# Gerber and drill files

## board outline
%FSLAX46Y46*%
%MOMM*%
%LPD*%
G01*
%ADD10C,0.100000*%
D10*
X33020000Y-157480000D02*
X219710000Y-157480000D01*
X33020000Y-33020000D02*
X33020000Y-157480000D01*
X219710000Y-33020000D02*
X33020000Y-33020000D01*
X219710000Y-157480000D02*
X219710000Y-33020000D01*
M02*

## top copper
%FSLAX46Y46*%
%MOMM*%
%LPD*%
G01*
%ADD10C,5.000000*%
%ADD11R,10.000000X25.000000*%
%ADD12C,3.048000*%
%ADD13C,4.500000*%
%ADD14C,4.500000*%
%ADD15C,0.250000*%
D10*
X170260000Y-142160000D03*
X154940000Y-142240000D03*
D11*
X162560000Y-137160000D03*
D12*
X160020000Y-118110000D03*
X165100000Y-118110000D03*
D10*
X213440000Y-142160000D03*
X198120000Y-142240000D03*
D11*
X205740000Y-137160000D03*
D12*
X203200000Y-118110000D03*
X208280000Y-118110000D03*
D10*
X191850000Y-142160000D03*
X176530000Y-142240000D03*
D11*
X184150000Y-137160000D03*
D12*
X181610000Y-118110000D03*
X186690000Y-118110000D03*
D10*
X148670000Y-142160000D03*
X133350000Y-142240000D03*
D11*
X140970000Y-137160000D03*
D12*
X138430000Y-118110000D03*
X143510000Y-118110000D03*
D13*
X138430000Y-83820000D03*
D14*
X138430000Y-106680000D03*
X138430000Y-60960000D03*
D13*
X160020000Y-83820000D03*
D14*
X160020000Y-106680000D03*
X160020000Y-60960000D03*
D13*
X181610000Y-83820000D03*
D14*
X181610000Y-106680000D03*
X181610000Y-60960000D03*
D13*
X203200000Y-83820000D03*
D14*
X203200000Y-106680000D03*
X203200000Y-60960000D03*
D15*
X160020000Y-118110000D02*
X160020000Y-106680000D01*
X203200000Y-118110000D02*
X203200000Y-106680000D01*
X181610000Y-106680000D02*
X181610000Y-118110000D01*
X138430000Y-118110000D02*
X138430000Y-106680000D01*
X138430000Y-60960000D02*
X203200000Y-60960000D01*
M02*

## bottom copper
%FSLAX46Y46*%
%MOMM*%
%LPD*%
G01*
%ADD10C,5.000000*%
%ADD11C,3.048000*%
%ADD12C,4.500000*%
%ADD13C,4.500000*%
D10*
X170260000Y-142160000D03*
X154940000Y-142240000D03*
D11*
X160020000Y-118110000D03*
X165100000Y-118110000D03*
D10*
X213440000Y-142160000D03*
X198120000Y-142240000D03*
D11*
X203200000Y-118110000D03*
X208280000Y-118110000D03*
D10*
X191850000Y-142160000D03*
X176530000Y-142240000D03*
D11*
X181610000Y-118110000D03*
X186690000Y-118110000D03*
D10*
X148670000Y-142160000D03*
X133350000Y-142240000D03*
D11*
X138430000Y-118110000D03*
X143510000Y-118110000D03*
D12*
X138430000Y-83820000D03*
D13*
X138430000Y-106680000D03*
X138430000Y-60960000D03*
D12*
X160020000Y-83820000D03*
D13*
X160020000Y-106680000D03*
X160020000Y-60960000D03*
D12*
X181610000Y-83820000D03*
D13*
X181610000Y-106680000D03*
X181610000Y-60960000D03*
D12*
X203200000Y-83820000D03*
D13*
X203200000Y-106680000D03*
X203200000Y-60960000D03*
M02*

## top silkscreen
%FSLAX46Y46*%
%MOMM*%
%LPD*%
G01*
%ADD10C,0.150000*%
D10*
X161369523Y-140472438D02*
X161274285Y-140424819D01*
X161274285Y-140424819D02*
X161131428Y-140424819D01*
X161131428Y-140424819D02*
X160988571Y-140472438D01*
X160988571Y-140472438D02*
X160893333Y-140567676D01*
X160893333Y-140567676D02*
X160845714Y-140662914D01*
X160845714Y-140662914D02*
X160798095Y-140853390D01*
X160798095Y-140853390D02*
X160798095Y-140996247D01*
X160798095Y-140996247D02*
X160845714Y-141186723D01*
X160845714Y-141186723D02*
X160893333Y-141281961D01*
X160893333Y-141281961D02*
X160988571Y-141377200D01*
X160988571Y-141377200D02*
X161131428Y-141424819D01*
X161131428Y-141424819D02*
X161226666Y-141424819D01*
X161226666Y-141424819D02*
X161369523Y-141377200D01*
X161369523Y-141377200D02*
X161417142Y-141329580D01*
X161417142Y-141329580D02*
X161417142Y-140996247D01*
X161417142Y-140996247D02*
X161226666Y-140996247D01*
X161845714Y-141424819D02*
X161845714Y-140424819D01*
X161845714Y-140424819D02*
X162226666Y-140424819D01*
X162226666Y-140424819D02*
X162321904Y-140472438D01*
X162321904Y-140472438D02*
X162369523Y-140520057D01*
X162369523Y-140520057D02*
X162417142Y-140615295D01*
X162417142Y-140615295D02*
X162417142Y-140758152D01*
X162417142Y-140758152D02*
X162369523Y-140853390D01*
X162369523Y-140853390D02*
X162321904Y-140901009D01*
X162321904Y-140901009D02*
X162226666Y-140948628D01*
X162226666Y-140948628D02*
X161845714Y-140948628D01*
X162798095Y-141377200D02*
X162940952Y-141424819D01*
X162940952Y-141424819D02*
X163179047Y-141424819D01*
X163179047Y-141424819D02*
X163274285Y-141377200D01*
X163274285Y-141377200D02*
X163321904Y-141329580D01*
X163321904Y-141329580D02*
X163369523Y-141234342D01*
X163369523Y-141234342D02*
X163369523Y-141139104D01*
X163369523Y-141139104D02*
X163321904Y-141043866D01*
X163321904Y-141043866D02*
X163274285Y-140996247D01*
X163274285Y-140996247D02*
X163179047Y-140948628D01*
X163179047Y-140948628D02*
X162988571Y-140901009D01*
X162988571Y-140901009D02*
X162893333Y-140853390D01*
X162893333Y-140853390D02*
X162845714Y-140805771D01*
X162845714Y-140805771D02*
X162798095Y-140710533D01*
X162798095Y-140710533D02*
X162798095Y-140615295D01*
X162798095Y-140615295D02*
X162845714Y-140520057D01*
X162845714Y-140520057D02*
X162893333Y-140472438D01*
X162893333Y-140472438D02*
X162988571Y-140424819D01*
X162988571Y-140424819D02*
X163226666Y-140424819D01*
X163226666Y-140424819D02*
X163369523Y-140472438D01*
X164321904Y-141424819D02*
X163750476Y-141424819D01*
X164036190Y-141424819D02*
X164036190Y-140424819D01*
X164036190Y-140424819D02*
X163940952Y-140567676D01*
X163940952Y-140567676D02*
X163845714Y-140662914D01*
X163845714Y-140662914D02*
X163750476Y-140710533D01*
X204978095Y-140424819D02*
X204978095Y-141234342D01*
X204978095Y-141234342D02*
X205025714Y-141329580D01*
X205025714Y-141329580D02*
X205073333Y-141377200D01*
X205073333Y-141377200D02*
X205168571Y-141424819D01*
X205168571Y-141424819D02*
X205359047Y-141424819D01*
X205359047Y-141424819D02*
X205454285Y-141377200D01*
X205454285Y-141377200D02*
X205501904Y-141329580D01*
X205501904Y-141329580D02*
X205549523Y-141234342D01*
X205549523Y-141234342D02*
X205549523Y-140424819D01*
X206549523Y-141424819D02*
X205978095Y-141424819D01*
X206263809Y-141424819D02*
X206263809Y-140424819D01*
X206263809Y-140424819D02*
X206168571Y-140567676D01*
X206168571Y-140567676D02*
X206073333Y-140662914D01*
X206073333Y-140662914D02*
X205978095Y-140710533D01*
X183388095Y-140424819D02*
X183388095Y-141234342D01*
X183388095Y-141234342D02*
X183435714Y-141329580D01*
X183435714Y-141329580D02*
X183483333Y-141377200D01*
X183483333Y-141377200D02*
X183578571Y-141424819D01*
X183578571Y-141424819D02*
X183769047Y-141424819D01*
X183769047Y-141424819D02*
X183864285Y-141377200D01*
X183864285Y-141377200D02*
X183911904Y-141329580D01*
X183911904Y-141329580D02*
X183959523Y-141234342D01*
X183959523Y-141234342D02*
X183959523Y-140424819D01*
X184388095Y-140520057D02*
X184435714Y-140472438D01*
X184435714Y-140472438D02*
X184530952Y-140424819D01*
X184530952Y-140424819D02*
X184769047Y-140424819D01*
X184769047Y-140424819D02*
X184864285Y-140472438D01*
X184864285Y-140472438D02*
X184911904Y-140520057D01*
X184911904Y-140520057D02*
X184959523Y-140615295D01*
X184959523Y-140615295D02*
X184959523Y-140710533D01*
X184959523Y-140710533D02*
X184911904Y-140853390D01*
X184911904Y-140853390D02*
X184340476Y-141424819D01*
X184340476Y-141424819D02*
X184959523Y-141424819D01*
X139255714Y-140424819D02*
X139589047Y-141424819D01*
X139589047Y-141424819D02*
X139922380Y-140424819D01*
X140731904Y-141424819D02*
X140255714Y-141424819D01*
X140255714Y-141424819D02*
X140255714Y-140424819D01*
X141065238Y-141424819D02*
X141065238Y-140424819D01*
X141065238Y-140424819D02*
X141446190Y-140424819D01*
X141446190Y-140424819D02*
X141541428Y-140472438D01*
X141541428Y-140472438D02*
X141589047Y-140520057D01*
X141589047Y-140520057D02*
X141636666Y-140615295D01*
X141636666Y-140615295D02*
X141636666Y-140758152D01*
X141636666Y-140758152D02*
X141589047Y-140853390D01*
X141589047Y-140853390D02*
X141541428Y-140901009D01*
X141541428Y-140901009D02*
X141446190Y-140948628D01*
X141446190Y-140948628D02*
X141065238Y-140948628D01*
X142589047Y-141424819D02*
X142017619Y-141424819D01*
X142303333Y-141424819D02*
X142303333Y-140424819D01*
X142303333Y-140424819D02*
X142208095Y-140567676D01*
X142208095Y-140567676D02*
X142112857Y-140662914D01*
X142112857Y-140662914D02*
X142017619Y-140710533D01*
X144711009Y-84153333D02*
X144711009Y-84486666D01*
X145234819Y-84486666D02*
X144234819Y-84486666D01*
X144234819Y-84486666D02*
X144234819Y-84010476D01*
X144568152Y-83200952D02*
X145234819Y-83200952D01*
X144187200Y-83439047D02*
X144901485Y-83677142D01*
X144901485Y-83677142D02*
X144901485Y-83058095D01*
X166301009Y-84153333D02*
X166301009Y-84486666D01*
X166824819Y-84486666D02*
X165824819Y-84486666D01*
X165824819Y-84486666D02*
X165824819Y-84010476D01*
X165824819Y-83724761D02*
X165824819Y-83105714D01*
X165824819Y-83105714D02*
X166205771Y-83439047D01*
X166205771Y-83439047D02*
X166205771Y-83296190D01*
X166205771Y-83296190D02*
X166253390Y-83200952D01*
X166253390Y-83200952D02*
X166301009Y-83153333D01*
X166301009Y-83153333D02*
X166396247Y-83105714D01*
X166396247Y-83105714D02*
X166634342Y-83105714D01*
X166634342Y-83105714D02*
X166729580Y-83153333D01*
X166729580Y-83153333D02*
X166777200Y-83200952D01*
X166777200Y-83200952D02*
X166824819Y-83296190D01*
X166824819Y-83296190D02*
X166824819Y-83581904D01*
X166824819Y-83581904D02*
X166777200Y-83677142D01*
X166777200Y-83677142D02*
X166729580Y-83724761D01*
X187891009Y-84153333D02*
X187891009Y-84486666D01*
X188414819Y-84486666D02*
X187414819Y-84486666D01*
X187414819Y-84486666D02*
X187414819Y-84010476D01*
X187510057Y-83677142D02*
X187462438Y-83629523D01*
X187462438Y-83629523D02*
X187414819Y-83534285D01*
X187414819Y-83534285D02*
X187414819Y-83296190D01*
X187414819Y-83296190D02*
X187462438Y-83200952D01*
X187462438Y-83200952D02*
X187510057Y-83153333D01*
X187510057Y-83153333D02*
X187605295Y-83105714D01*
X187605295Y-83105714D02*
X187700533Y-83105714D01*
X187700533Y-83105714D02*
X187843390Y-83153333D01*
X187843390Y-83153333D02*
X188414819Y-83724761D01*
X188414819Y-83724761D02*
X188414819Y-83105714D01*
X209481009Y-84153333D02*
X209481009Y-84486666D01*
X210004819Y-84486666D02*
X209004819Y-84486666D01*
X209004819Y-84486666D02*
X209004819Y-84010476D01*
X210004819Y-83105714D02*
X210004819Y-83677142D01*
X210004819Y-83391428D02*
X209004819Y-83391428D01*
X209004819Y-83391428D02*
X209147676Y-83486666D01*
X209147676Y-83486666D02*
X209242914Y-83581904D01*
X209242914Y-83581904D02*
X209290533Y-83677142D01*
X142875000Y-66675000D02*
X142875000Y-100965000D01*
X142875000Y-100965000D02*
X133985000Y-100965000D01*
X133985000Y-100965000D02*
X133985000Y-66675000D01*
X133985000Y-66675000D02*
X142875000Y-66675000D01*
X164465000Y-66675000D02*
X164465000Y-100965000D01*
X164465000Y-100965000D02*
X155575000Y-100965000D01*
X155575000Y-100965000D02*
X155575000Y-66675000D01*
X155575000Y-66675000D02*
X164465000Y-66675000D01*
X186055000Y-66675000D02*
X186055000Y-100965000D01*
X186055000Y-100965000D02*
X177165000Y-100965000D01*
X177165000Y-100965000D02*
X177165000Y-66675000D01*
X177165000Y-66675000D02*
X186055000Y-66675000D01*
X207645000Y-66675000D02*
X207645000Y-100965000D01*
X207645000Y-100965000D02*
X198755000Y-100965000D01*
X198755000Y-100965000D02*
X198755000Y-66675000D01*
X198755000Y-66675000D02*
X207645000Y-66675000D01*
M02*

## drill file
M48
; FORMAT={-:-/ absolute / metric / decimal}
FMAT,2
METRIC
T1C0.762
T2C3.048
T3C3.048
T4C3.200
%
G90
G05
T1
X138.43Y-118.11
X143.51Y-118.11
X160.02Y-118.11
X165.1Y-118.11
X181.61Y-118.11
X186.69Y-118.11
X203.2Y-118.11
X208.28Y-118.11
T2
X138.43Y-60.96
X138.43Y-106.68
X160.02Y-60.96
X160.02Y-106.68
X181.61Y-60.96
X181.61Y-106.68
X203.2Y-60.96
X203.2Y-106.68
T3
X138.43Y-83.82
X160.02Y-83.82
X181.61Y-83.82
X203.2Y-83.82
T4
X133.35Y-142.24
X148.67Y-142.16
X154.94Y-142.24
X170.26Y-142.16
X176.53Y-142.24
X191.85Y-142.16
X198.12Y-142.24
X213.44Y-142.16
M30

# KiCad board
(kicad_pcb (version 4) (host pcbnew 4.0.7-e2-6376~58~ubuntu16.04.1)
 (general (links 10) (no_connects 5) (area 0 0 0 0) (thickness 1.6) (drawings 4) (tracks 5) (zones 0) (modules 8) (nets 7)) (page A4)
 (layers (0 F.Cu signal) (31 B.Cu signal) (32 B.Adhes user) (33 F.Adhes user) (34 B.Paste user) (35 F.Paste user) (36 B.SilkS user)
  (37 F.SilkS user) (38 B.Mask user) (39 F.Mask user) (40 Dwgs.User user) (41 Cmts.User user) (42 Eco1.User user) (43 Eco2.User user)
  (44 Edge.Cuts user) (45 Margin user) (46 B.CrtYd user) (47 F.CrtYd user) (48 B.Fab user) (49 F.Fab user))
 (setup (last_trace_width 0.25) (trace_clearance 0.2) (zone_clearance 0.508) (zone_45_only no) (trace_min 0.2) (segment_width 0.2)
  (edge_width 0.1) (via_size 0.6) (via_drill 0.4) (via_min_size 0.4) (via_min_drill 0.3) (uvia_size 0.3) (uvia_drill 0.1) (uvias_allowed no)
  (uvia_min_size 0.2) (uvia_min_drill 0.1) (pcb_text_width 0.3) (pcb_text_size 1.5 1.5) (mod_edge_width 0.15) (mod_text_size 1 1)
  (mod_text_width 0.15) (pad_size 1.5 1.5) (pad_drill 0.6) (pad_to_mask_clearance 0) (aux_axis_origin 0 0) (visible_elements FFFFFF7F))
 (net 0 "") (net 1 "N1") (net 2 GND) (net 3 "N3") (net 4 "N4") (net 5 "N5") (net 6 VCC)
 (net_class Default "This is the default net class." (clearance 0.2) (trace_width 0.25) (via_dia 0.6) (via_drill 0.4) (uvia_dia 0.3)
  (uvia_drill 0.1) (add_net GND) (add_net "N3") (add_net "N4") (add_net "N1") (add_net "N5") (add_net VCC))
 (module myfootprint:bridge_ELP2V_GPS (layer F.Cu) (at 162.56 137.16)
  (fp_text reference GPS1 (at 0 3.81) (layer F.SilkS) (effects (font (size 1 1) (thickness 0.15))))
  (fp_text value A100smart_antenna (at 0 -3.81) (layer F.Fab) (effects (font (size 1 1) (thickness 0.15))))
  (pad "" np_thru_hole circle (at 7.7 5) (size 5 5) (drill 3.2) (layers *.Cu *.Mask))
  (pad "" np_thru_hole circle (at -7.62 5.08) (size 5 5) (drill 3.2) (layers *.Cu *.Mask))
  (pad "" connect rect (at 0 0) (size 10 25) (layers F.Cu F.Mask))
  (pad 10 thru_hole circle (at -2.54 -19.05) (size 3.048 3.048) (drill 0.762) (layers *.Mask F.Cu) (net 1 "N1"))
  (pad 11 thru_hole circle (at 2.54 -19.05) (size 3.048 3.048) (drill 0.762) (layers *.Mask B.Cu) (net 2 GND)))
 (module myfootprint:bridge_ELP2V (layer F.Cu) (at 205.74 137.16)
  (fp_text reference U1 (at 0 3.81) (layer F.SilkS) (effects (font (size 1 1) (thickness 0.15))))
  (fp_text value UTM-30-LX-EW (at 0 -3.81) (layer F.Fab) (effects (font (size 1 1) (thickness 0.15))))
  (pad "" np_thru_hole circle (at 7.7 5) (size 5 5) (drill 3.2) (layers *.Cu *.Mask))
  (pad "" np_thru_hole circle (at -7.62 5.08) (size 5 5) (drill 3.2) (layers *.Cu *.Mask))
  (pad "" connect rect (at 0 0) (size 10 25) (layers F.Cu F.Mask))
  (pad 1 thru_hole circle (at -2.54 -19.05) (size 3.048 3.048) (drill 0.762) (layers *.Mask F.Cu) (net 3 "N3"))
  (pad 2 thru_hole circle (at 2.54 -19.05) (size 3.048 3.048) (drill 0.762) (layers *.Mask B.Cu) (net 2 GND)))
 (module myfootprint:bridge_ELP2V (layer F.Cu) (at 184.15 137.16)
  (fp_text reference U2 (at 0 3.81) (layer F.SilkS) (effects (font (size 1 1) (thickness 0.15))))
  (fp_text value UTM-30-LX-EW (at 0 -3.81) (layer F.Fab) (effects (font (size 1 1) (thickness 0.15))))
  (pad "" np_thru_hole circle (at 7.7 5) (size 5 5) (drill 3.2) (layers *.Cu *.Mask))
  (pad "" np_thru_hole circle (at -7.62 5.08) (size 5 5) (drill 3.2) (layers *.Cu *.Mask))
  (pad "" connect rect (at 0 0) (size 10 25) (layers F.Cu F.Mask))
  (pad 1 thru_hole circle (at -2.54 -19.05) (size 3.048 3.048) (drill 0.762) (layers *.Mask F.Cu) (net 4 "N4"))
  (pad 2 thru_hole circle (at 2.54 -19.05) (size 3.048 3.048) (drill 0.762) (layers *.Mask B.Cu) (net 2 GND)))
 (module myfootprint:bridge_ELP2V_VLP (layer F.Cu) (at 140.97 137.16)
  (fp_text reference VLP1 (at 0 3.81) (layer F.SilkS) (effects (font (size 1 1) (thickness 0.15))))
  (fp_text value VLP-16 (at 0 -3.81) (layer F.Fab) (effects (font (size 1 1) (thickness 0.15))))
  (pad "" np_thru_hole circle (at 7.7 5) (size 5 5) (drill 3.2) (layers *.Cu *.Mask))
  (pad "" np_thru_hole circle (at -7.62 5.08) (size 5 5) (drill 3.2) (layers *.Cu *.Mask))
  (pad "" connect rect (at 0 0) (size 10 25) (layers F.Cu F.Mask))
  (pad 2 thru_hole circle (at -2.54 -19.05) (size 3.048 3.048) (drill 0.762) (layers *.Mask F.Cu) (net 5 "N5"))
  (pad 1 thru_hole circle (at 2.54 -19.05) (size 3.048 3.048) (drill 0.762) (layers *.Mask B.Cu) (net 2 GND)))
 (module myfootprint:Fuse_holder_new (layer F.Cu) (at 143.51 83.82 270)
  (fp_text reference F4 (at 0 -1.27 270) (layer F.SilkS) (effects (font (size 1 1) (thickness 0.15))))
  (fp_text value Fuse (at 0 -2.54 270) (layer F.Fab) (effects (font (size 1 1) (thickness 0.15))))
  (fp_line (start -17.145 0.635) (end 17.145 0.635) (layer F.SilkS) (width 0.15))
  (fp_line (start 17.145 0.635) (end 17.145 9.525) (layer F.SilkS) (width 0.15))
  (fp_line (start 17.145 9.525) (end -17.145 9.525) (layer F.SilkS) (width 0.15))
  (fp_line (start -17.145 9.525) (end -17.145 0.635) (layer F.SilkS) (width 0.15))
  (pad "" np_thru_hole circle (at 0 5.08 270) (size 4.5 4.5) (drill 3.048) (layers *.Cu *.Mask))
  (pad 1 thru_hole circle (at 22.86 5.08 270) (size 4.5 4.5) (drill 3.048) (layers *.Mask F.Cu) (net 5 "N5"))
  (pad 2 thru_hole circle (at -22.86 5.08 270) (size 4.5 4.5) (drill 3.048) (layers *.Mask F.Cu) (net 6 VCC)))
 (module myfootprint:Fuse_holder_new (layer F.Cu) (at 165.1 83.82 270)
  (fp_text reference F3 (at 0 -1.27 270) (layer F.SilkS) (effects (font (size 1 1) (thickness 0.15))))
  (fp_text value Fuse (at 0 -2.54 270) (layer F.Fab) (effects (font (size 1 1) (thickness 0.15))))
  (fp_line (start -17.145 0.635) (end 17.145 0.635) (layer F.SilkS) (width 0.15))
  (fp_line (start 17.145 0.635) (end 17.145 9.525) (layer F.SilkS) (width 0.15))
  (fp_line (start 17.145 9.525) (end -17.145 9.525) (layer F.SilkS) (width 0.15))
  (fp_line (start -17.145 9.525) (end -17.145 0.635) (layer F.SilkS) (width 0.15))
  (pad "" np_thru_hole circle (at 0 5.08 270) (size 4.5 4.5) (drill 3.048) (layers *.Cu *.Mask))
  (pad 1 thru_hole circle (at 22.86 5.08 270) (size 4.5 4.5) (drill 3.048) (layers *.Mask F.Cu) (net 1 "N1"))
  (pad 2 thru_hole circle (at -22.86 5.08 270) (size 4.5 4.5) (drill 3.048) (layers *.Mask F.Cu) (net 6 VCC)))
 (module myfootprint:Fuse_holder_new (layer F.Cu) (at 186.69 83.82 270)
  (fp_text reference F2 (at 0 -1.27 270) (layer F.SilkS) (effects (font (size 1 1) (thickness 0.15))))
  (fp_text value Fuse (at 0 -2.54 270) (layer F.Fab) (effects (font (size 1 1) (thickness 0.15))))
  (fp_line (start -17.145 0.635) (end 17.145 0.635) (layer F.SilkS) (width 0.15))
  (fp_line (start 17.145 0.635) (end 17.145 9.525) (layer F.SilkS) (width 0.15))
  (fp_line (start 17.145 9.525) (end -17.145 9.525) (layer F.SilkS) (width 0.15))
  (fp_line (start -17.145 9.525) (end -17.145 0.635) (layer F.SilkS) (width 0.15))
  (pad "" np_thru_hole circle (at 0 5.08 270) (size 4.5 4.5) (drill 3.048) (layers *.Cu *.Mask))
  (pad 1 thru_hole circle (at 22.86 5.08 270) (size 4.5 4.5) (drill 3.048) (layers *.Mask F.Cu) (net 4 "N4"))
  (pad 2 thru_hole circle (at -22.86 5.08 270) (size 4.5 4.5) (drill 3.048) (layers *.Mask F.Cu) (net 6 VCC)))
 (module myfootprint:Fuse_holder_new (layer F.Cu) (at 208.28 83.82 270)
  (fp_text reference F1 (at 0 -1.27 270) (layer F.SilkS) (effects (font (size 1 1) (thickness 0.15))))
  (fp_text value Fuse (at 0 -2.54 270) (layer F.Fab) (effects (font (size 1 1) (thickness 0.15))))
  (fp_line (start -17.145 0.635) (end 17.145 0.635) (layer F.SilkS) (width 0.15))
  (fp_line (start 17.145 0.635) (end 17.145 9.525) (layer F.SilkS) (width 0.15))
  (fp_line (start 17.145 9.525) (end -17.145 9.525) (layer F.SilkS) (width 0.15))
  (fp_line (start -17.145 9.525) (end -17.145 0.635) (layer F.SilkS) (width 0.15))
  (pad "" np_thru_hole circle (at 0 5.08 270) (size 4.5 4.5) (drill 3.048) (layers *.Cu *.Mask))
  (pad 1 thru_hole circle (at 22.86 5.08 270) (size 4.5 4.5) (drill 3.048) (layers *.Mask F.Cu) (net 3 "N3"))
  (pad 2 thru_hole circle (at -22.86 5.08 270) (size 4.5 4.5) (drill 3.048) (layers *.Mask F.Cu) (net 6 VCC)))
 (gr_line (start 33.02 157.48) (end 219.71 157.48) (angle 90) (layer Edge.Cuts) (width 0.1))
 (gr_line (start 33.02 33.02) (end 33.02 157.48) (angle 90) (layer Edge.Cuts) (width 0.1))
 (gr_line (start 219.71 33.02) (end 33.02 33.02) (angle 90) (layer Edge.Cuts) (width 0.1))
 (gr_line (start 219.71 157.48) (end 219.71 33.02) (angle 90) (layer Edge.Cuts) (width 0.1))
 (segment (start 160.02 118.11) (end 160.02 106.68) (width 0.25) (layer F.Cu) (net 1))
 (segment (start 203.2 118.11) (end 203.2 106.68) (width 0.25) (layer F.Cu) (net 3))
 (segment (start 181.61 106.68) (end 181.61 118.11) (width 0.25) (layer F.Cu) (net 4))
 (segment (start 138.43 118.11) (end 138.43 106.68) (width 0.25) (layer F.Cu) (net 5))
 (segment (start 138.43 60.96) (end 203.2 60.96) (width 0.25) (layer F.Cu) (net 6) (status C00000)))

